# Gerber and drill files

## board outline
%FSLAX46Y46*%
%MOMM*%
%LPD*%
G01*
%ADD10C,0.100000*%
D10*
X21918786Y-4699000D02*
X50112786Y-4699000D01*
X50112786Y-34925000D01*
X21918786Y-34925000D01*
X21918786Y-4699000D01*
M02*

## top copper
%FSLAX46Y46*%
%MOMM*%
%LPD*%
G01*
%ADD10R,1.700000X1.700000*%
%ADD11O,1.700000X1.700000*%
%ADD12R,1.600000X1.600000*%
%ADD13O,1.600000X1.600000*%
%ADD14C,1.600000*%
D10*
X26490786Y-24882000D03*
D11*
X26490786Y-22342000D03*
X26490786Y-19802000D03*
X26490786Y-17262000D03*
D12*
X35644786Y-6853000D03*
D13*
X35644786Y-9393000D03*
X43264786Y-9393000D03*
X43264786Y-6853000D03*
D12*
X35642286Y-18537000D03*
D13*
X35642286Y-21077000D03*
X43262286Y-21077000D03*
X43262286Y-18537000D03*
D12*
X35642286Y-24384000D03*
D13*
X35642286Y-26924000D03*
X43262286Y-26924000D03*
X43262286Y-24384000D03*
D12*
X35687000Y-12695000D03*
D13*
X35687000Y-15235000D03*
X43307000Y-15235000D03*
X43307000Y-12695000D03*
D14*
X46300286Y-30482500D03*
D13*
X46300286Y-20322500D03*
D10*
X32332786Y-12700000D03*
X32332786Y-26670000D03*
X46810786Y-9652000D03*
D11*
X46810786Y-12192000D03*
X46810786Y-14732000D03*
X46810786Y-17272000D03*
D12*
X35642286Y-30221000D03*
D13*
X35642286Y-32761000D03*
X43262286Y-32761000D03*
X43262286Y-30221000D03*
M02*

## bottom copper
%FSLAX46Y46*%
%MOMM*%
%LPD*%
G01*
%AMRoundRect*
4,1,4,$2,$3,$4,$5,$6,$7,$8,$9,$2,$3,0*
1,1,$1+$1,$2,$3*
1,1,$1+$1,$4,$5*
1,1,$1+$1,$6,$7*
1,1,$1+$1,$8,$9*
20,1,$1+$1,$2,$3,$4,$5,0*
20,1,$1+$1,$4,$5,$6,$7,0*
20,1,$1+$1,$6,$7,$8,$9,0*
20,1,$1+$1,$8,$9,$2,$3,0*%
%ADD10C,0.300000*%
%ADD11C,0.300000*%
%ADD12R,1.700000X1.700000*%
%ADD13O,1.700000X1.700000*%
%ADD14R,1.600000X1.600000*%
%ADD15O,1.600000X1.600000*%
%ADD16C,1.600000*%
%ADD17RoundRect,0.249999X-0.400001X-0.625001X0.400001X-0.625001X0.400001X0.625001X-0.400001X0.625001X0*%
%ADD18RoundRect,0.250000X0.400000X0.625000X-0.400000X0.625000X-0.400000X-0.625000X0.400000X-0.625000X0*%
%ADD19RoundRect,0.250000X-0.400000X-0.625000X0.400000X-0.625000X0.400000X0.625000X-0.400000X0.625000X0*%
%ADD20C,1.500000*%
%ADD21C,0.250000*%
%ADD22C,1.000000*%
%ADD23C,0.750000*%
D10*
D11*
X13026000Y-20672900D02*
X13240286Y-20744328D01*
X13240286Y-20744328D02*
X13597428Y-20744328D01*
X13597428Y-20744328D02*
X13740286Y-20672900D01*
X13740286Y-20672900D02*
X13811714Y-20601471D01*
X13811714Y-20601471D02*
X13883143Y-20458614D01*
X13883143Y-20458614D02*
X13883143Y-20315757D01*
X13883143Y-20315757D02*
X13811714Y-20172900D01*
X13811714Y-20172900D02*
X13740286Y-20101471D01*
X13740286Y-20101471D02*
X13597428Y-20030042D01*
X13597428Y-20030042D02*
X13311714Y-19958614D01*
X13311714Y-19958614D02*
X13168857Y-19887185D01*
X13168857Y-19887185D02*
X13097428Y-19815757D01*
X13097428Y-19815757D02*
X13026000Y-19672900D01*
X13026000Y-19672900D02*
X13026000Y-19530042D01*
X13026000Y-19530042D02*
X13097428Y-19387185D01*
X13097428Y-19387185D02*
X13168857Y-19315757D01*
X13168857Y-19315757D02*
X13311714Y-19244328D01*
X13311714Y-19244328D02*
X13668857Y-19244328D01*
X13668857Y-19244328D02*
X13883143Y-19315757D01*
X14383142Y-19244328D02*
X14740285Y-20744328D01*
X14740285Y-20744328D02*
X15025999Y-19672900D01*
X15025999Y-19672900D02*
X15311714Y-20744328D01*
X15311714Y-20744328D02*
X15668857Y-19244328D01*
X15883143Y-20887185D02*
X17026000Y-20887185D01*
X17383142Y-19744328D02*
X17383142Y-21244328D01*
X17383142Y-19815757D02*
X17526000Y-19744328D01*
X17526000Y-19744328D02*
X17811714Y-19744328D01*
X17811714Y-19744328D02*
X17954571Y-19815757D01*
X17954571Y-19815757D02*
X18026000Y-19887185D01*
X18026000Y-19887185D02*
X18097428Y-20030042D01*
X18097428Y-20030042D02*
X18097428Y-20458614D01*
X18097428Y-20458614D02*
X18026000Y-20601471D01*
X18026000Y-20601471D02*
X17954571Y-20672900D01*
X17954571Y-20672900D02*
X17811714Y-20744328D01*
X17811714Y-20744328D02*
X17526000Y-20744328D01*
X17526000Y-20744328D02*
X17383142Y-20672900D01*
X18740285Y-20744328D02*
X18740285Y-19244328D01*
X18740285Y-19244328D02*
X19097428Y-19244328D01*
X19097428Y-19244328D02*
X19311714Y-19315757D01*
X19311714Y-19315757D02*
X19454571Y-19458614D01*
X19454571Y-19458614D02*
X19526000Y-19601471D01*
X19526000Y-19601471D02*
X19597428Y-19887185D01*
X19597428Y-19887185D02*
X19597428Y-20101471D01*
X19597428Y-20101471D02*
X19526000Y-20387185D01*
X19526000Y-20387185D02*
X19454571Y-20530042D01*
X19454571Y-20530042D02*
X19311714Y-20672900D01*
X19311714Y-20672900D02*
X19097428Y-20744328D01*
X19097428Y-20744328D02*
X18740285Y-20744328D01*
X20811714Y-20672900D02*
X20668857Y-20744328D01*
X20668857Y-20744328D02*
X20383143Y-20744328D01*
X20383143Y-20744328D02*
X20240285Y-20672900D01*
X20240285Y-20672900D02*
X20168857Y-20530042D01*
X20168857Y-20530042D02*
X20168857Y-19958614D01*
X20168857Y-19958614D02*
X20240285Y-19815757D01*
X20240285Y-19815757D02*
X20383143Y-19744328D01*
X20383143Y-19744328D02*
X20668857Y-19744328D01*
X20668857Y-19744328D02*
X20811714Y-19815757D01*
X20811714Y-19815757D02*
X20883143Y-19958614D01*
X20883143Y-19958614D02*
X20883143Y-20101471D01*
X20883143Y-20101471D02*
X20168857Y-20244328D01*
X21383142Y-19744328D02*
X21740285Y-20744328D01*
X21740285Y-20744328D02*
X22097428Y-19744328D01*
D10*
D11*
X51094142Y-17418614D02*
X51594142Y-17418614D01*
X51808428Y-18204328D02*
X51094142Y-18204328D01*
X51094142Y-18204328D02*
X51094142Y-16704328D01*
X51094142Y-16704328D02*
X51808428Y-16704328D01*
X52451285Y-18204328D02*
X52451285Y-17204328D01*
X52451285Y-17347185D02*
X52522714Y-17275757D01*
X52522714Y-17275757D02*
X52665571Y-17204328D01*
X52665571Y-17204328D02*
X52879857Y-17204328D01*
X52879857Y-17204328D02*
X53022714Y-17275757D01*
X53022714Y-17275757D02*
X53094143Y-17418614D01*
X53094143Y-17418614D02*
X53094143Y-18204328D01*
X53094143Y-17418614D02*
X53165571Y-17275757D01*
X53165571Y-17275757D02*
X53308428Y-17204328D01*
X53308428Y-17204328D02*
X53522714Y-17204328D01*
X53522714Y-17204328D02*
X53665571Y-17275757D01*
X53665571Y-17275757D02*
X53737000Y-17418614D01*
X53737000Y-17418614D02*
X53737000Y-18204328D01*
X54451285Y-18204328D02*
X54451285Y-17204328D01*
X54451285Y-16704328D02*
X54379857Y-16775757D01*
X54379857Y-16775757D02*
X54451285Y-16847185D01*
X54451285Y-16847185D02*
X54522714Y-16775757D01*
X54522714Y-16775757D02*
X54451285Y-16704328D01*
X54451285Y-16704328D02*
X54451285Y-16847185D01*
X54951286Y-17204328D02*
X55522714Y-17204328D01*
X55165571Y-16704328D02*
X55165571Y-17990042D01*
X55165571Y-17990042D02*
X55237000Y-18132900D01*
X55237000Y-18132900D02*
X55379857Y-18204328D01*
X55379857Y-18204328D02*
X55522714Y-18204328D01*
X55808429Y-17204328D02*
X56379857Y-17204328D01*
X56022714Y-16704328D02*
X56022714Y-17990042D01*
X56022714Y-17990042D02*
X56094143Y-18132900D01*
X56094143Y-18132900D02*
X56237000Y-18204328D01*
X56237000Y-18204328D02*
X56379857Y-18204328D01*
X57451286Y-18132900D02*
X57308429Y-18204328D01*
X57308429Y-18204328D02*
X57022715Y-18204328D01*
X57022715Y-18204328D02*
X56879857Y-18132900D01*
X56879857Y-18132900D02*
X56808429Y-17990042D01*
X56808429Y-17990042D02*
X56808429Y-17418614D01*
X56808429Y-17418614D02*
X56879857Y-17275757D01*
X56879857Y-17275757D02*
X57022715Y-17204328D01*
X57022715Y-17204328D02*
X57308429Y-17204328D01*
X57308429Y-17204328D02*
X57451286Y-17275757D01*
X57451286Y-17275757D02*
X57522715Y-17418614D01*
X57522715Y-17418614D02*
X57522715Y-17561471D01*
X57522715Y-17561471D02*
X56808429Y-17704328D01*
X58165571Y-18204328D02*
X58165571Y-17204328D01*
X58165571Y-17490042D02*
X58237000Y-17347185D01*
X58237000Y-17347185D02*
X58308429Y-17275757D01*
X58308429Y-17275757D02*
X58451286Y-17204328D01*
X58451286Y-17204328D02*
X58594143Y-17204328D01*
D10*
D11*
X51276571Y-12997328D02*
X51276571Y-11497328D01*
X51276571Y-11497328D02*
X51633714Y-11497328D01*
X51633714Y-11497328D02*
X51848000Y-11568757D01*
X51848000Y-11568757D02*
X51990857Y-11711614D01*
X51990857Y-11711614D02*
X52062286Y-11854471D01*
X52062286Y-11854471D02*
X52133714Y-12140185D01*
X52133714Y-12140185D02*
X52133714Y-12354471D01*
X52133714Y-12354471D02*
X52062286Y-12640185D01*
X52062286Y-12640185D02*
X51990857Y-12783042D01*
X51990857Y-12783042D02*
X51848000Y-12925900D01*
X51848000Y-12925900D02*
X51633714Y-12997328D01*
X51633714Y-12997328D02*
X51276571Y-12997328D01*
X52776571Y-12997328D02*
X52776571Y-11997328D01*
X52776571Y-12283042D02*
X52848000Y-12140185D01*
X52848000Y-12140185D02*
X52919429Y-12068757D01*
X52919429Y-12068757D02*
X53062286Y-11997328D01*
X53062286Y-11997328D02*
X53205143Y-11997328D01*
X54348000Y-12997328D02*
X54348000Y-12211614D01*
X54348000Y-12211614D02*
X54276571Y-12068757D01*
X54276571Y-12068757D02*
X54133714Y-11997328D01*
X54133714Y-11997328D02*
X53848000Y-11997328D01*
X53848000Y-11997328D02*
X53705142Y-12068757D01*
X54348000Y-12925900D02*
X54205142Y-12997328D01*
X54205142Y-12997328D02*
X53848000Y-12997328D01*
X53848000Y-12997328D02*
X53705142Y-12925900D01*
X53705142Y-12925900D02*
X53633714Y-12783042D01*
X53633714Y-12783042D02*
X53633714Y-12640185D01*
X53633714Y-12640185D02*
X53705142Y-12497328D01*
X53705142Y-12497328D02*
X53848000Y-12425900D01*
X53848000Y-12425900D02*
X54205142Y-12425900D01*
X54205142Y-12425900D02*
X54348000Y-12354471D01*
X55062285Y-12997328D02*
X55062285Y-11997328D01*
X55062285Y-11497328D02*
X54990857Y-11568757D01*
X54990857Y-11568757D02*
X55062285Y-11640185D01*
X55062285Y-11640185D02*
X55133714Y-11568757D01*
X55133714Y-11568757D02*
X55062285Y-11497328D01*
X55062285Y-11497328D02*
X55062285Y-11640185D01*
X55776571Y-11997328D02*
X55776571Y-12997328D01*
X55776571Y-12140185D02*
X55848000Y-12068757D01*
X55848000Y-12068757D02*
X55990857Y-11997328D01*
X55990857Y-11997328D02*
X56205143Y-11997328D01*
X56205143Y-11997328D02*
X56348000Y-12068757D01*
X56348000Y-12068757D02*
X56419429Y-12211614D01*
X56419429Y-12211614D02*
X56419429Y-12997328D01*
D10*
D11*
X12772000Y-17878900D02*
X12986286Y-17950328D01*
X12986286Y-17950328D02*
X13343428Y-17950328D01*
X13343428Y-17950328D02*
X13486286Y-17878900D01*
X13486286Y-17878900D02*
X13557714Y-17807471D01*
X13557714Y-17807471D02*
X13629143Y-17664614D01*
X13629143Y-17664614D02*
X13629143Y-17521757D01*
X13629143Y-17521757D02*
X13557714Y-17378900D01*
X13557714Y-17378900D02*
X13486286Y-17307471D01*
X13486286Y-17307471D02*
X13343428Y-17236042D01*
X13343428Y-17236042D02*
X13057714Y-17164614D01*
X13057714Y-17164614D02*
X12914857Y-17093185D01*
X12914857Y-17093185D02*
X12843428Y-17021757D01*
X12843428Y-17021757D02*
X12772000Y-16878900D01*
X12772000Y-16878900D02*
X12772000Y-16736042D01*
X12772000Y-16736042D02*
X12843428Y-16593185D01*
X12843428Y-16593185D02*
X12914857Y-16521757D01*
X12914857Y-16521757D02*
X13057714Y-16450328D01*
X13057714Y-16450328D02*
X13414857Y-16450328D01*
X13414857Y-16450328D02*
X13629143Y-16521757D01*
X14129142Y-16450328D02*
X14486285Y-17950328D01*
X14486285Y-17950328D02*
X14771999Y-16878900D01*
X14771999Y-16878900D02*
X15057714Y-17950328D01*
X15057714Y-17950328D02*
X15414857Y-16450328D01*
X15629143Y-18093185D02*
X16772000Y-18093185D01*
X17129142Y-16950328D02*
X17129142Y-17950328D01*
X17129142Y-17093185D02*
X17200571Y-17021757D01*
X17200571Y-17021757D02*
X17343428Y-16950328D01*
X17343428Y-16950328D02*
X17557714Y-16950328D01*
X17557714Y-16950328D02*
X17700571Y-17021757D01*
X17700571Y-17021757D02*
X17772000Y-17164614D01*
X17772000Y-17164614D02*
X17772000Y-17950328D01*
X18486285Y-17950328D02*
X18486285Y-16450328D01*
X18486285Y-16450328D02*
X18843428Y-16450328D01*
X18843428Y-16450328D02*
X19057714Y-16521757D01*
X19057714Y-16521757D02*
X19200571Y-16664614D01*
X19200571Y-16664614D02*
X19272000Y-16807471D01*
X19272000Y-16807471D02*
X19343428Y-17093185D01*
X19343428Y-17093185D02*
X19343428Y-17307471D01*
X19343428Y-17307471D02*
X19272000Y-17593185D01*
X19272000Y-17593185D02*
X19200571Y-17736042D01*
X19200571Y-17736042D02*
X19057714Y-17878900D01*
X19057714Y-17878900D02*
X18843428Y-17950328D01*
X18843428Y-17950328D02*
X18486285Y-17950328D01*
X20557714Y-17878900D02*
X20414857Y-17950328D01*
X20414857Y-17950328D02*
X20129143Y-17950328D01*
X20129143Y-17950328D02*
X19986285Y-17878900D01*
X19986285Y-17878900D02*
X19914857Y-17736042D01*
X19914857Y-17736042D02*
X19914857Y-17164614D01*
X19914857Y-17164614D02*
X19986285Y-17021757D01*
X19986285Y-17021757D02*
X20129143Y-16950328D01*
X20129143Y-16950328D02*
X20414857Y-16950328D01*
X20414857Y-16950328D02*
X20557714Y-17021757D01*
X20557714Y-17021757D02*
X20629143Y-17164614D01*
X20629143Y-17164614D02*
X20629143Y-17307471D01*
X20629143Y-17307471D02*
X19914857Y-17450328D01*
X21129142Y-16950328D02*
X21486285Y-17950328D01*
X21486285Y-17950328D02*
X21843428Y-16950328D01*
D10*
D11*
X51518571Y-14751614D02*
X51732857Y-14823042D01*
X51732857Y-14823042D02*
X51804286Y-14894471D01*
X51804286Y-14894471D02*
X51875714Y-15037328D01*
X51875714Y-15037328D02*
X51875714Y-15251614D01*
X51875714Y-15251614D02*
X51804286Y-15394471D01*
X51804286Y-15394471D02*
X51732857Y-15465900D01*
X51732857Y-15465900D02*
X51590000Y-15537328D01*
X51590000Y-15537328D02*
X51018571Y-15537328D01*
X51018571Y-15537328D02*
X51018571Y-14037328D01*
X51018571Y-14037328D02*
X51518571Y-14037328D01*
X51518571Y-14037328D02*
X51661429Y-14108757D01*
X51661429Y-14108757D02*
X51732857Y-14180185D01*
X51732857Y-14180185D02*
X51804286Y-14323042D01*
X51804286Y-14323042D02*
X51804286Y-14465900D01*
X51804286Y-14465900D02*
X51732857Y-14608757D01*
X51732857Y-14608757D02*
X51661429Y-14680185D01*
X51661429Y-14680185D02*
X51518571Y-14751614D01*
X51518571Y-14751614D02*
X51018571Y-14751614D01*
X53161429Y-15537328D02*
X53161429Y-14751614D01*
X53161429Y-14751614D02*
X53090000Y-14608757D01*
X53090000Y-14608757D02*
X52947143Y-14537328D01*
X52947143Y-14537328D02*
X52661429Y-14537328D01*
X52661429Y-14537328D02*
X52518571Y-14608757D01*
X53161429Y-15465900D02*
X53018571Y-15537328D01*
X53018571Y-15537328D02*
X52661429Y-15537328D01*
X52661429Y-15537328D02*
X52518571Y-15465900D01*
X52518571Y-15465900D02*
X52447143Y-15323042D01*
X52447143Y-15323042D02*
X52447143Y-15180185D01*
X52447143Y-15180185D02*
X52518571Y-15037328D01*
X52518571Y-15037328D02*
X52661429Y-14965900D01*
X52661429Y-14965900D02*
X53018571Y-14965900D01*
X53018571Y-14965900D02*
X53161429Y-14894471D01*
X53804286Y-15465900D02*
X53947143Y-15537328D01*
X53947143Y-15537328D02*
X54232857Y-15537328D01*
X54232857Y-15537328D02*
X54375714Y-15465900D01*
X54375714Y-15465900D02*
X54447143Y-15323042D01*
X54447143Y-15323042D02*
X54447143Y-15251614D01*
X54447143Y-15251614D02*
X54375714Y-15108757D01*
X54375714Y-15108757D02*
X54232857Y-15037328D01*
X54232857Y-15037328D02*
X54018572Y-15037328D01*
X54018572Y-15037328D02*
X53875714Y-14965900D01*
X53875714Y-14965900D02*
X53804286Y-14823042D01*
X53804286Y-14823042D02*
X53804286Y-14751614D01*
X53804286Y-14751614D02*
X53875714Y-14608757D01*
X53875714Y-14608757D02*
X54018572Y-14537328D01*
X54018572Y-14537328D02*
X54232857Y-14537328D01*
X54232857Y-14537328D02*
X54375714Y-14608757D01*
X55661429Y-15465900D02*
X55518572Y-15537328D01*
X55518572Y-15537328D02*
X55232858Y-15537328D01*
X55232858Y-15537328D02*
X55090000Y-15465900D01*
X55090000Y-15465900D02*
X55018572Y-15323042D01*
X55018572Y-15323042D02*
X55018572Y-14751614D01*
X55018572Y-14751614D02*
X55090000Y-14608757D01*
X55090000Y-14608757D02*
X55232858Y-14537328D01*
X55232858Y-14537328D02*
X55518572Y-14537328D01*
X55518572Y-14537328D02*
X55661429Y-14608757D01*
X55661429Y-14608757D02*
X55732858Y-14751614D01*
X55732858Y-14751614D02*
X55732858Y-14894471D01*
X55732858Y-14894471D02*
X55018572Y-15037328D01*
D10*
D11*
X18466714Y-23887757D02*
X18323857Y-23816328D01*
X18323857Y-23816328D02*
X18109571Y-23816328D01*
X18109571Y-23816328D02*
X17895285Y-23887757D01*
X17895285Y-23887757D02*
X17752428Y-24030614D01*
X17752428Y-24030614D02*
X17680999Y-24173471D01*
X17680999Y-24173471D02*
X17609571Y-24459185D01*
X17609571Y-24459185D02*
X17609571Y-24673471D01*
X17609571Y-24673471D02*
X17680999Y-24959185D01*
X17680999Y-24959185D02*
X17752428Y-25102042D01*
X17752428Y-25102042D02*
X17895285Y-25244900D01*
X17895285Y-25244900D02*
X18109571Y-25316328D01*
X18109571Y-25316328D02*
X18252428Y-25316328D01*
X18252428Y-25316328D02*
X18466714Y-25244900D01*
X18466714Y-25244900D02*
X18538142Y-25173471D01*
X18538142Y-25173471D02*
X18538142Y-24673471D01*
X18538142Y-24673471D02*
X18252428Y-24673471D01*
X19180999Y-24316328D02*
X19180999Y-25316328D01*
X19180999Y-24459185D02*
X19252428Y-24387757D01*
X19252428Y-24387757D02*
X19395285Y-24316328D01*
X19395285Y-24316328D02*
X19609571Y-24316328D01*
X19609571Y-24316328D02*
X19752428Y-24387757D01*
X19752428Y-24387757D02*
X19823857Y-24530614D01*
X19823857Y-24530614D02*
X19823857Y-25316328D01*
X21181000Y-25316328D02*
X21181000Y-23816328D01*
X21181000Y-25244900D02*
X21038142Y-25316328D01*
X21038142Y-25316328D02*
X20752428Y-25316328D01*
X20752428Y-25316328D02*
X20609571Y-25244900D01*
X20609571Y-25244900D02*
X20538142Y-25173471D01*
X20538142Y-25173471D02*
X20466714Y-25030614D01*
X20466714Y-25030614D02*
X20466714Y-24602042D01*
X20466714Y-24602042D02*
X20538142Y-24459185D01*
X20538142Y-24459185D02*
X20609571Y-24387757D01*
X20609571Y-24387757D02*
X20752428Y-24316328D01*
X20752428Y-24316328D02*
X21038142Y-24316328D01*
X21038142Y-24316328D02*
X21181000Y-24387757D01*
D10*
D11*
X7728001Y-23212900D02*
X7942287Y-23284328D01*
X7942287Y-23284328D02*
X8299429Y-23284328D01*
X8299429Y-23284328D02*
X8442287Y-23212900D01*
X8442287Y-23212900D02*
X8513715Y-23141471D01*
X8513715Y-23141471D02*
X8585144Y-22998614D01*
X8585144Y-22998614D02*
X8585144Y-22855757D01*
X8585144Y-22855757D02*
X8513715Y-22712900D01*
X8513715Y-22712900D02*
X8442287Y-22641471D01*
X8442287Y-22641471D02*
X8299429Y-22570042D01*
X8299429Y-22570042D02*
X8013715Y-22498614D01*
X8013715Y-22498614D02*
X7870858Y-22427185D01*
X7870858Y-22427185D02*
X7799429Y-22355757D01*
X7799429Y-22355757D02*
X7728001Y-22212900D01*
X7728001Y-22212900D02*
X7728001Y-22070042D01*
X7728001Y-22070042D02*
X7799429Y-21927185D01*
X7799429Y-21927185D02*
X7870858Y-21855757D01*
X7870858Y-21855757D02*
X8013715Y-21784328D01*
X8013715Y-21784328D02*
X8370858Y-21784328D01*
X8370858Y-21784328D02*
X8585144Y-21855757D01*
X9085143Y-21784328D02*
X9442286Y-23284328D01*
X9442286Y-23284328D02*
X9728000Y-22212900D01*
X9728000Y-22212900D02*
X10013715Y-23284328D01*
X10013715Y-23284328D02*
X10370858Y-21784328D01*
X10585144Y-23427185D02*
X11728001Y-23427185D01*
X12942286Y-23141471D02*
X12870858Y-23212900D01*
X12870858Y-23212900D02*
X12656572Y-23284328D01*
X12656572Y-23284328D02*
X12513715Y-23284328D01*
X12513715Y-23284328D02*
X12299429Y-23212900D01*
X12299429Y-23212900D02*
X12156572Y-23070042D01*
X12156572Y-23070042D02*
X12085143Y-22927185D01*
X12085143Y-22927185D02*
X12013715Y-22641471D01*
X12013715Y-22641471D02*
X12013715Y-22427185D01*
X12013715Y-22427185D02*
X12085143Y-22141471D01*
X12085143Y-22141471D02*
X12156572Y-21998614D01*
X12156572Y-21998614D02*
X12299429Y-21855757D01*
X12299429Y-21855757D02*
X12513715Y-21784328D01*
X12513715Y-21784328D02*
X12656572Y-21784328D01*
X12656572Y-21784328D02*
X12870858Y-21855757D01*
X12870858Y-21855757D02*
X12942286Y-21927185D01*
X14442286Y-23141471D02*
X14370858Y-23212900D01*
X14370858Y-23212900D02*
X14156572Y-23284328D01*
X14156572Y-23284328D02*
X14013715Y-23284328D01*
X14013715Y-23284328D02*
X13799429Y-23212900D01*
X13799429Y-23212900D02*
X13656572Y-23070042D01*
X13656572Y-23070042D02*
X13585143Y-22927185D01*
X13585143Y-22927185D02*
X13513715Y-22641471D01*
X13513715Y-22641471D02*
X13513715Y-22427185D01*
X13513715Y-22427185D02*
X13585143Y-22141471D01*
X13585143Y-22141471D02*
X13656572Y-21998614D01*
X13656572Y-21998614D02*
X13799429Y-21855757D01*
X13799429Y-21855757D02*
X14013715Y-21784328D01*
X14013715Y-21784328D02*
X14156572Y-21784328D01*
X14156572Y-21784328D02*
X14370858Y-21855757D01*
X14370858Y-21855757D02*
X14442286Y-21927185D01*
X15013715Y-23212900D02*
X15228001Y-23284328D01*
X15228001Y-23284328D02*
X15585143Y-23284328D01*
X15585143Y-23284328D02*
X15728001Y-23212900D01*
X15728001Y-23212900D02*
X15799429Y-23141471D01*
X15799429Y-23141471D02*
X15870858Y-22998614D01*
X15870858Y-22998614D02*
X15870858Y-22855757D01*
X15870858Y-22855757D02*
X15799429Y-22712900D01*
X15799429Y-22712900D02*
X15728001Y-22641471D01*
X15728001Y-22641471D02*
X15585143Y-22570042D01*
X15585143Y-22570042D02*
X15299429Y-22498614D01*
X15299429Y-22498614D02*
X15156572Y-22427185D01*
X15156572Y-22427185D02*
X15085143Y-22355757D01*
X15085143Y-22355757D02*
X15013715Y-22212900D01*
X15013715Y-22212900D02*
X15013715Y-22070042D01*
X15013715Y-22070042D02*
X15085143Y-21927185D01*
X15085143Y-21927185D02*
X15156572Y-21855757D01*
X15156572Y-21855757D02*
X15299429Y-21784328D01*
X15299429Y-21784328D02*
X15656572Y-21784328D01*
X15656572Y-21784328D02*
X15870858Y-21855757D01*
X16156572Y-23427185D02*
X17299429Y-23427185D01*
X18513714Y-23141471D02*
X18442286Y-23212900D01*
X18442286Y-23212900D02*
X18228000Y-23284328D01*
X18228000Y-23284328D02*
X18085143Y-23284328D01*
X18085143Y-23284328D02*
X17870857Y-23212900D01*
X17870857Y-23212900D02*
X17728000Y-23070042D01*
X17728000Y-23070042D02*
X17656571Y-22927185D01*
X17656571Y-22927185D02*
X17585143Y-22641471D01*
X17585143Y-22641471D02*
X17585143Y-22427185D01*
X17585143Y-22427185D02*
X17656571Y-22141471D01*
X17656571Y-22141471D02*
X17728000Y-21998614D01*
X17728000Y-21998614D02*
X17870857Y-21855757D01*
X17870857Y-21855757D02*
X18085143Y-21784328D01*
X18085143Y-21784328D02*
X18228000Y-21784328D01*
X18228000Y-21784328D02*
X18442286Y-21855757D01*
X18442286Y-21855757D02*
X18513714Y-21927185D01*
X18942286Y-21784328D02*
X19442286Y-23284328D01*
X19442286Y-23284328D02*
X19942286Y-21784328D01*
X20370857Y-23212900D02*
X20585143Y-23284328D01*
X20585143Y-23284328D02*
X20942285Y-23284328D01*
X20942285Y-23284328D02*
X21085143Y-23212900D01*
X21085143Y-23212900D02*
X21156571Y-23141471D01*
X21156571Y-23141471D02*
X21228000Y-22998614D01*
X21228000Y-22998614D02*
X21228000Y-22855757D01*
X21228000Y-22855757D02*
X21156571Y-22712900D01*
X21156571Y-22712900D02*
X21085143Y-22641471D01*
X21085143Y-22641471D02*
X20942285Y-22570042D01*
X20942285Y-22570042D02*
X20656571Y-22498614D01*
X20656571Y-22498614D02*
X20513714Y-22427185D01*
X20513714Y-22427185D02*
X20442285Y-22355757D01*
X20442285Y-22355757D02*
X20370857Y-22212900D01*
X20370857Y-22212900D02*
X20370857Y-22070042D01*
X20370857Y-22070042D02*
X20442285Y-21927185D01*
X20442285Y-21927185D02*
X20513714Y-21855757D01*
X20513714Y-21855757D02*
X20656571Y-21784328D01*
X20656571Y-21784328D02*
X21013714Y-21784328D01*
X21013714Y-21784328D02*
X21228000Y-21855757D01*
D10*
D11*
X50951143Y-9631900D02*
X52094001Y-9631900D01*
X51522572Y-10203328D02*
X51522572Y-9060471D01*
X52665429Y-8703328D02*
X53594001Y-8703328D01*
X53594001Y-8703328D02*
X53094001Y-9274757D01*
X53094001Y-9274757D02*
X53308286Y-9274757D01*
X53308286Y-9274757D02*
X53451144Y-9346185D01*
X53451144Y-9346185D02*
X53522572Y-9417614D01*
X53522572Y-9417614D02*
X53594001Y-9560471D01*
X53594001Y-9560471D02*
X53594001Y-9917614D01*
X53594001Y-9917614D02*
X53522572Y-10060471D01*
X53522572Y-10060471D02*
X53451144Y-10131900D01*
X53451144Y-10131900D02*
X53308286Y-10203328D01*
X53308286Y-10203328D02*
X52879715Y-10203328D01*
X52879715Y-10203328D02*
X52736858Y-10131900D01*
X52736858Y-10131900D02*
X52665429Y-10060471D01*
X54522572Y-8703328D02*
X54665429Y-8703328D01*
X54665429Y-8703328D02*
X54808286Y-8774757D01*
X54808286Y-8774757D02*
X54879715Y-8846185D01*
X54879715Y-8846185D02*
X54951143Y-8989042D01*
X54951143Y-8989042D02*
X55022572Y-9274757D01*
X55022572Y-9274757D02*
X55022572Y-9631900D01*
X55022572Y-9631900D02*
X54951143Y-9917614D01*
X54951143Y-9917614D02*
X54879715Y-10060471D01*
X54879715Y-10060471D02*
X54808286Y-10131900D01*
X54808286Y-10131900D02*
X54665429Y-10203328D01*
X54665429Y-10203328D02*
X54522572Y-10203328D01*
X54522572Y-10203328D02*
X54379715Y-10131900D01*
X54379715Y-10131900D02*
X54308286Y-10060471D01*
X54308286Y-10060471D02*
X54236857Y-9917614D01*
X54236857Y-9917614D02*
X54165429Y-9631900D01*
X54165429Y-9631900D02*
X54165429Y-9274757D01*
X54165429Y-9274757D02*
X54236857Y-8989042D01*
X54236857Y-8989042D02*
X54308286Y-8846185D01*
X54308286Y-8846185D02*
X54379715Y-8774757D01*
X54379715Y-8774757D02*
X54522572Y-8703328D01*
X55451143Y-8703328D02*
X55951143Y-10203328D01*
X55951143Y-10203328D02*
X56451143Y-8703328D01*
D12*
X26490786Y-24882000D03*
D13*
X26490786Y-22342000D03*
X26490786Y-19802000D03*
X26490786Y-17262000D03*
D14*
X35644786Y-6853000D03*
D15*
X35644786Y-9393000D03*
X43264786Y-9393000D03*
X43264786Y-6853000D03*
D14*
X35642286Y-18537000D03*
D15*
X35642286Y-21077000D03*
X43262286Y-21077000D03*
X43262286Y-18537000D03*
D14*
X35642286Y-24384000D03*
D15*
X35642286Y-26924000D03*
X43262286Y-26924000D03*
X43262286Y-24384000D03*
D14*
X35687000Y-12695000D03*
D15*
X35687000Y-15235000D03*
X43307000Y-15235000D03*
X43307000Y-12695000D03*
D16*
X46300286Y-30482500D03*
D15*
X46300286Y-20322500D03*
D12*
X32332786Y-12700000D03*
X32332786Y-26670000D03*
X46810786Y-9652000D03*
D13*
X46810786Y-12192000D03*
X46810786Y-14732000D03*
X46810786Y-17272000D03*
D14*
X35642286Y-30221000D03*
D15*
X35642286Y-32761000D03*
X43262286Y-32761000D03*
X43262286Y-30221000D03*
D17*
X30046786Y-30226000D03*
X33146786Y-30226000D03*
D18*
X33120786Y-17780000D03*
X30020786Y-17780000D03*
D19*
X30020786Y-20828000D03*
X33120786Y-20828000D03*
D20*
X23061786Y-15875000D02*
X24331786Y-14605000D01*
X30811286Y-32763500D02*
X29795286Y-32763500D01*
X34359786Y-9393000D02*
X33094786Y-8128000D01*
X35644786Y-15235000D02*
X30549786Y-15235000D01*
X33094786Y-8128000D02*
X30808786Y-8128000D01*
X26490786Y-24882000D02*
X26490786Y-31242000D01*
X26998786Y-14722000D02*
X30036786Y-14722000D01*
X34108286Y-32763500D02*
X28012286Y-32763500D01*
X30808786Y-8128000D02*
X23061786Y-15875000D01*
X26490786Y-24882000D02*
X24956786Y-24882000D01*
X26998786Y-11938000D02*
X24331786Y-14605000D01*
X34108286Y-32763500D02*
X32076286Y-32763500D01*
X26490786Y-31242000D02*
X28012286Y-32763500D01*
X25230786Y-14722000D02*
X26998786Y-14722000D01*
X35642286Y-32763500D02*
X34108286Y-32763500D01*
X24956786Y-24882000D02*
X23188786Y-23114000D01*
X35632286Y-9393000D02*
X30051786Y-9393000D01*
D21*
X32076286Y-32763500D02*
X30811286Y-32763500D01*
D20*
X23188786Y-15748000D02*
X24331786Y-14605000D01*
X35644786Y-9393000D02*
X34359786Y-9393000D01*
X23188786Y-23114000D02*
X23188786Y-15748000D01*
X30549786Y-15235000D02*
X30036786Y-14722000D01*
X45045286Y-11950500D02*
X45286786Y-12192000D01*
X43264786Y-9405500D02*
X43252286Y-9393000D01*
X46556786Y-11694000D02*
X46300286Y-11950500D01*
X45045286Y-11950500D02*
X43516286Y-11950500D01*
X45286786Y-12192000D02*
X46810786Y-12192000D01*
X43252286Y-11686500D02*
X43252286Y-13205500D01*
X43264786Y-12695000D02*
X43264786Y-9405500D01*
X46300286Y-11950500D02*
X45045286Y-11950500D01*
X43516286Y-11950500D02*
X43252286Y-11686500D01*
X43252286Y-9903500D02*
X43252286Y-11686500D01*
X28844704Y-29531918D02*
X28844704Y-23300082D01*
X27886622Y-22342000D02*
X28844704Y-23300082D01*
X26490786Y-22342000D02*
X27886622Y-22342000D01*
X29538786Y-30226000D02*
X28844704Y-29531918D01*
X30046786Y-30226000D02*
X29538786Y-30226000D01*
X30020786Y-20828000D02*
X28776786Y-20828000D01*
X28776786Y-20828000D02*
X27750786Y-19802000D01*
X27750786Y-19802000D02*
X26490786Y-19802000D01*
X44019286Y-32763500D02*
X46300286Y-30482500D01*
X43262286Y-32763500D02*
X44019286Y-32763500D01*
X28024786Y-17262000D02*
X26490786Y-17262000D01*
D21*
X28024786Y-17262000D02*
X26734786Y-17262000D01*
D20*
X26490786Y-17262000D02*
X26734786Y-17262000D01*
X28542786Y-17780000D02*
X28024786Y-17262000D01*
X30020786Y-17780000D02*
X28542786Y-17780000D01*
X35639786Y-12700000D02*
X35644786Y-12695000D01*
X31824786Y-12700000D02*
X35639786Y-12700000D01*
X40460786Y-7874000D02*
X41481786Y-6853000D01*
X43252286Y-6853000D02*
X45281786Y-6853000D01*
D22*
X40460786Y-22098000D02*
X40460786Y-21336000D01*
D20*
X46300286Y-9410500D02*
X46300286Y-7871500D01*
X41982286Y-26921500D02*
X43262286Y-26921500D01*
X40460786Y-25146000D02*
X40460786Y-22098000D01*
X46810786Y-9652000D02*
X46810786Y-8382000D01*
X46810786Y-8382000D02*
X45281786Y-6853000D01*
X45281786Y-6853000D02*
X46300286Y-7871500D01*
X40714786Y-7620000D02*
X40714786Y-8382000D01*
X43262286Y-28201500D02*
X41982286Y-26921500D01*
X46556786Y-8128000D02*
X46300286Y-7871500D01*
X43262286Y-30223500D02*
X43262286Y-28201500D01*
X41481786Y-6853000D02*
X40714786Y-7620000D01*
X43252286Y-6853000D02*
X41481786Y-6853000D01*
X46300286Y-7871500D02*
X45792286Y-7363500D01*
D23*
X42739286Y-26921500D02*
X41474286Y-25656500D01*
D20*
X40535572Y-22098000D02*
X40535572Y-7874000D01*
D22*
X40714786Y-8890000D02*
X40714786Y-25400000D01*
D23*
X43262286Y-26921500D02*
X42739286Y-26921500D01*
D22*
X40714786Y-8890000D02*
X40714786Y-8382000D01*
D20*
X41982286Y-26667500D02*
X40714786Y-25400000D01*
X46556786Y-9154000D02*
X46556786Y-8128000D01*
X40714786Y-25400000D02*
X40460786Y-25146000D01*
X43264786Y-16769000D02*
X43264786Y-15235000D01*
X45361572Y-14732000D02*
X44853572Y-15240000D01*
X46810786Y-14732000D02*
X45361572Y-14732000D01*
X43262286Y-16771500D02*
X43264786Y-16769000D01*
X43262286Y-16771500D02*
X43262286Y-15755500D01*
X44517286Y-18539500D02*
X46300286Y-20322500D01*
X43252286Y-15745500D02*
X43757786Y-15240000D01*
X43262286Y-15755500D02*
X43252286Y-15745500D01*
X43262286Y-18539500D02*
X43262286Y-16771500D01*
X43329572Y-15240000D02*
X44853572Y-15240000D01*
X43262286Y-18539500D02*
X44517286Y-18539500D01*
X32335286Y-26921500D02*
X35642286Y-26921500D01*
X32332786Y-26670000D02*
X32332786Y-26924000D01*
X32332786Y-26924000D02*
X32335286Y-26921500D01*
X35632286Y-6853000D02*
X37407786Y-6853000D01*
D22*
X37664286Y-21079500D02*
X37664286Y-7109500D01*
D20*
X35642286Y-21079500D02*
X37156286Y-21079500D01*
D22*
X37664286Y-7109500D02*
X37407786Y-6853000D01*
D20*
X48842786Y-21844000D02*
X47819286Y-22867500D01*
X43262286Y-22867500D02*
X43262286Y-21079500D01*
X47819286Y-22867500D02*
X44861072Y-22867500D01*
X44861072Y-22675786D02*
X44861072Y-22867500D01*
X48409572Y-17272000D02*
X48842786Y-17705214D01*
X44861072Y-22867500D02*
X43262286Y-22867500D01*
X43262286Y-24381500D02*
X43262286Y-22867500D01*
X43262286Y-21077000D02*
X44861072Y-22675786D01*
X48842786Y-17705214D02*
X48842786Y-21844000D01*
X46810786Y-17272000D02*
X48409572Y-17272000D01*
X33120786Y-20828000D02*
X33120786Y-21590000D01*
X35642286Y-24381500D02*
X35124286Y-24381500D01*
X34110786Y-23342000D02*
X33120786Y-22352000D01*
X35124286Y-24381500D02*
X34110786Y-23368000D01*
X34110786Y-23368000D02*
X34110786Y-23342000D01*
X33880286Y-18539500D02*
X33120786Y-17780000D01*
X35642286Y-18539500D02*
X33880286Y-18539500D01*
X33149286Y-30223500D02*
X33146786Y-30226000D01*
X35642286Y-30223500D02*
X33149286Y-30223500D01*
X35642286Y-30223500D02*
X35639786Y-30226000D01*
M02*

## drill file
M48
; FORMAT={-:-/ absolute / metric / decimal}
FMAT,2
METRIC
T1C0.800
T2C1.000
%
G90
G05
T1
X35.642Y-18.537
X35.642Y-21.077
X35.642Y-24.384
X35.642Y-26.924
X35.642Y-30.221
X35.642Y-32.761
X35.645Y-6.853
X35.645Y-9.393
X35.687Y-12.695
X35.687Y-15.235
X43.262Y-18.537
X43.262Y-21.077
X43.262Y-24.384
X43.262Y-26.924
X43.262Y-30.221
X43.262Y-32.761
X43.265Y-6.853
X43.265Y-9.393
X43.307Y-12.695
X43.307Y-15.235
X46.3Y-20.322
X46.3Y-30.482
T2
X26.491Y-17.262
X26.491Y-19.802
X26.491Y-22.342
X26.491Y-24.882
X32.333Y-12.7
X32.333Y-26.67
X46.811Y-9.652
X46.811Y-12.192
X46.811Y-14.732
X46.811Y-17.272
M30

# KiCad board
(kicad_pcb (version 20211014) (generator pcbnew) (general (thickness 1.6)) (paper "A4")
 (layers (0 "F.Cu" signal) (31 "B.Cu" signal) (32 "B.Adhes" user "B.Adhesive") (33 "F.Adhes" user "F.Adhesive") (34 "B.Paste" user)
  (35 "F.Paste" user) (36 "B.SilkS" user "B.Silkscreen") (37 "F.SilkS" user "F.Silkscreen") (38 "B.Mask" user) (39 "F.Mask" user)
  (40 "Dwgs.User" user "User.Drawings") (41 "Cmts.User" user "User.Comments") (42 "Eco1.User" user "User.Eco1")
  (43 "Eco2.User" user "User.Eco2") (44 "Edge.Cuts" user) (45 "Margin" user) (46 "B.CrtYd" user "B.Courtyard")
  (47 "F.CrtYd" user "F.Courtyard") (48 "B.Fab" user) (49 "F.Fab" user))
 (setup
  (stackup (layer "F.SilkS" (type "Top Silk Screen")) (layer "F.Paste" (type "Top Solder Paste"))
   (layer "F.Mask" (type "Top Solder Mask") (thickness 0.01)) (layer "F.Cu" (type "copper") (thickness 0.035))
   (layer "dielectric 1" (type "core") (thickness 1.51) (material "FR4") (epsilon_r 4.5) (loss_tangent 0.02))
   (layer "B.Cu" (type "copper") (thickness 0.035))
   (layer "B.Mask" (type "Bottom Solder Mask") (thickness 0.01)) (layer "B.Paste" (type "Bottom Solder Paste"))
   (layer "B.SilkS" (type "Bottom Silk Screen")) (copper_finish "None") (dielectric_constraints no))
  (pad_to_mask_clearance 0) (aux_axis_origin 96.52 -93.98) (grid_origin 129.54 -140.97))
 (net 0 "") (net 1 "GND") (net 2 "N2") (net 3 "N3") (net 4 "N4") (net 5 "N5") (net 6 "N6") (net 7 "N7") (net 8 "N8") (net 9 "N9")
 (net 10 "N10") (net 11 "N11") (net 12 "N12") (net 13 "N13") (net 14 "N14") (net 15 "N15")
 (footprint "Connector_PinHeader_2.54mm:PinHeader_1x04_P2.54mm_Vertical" (layer "F.Cu") (at 26.490786 24.882 180)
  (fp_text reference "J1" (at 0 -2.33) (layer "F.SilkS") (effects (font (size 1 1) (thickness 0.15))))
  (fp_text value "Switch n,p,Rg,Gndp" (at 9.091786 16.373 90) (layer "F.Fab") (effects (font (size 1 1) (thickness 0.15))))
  (pad "1" thru_hole rect (at 0 0 180) (size 1.7 1.7) (drill 1) (layers *.Cu *.Mask) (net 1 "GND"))
  (pad "2" thru_hole oval (at 0 2.54 180) (size 1.7 1.7) (drill 1) (layers *.Cu *.Mask) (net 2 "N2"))
  (pad "3" thru_hole oval (at 0 5.08 180) (size 1.7 1.7) (drill 1) (layers *.Cu *.Mask) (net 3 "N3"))
  (pad "4" thru_hole oval (at 0 7.62 180) (size 1.7 1.7) (drill 1) (layers *.Cu *.Mask) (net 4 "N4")))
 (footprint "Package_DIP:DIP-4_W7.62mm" (layer "F.Cu") (at 35.644786 6.853)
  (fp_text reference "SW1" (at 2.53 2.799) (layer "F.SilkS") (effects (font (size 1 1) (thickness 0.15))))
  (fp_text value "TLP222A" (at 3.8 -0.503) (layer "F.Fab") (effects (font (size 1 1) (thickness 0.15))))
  (pad "1" thru_hole rect locked (at 0 0) (size 1.6 1.6) (drill 0.8) (layers *.Cu *.Mask) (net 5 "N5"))
  (pad "2" thru_hole oval locked (at 0 2.54) (size 1.6 1.6) (drill 0.8) (layers *.Cu *.Mask) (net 1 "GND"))
  (pad "3" thru_hole oval locked (at 7.62 2.54) (size 1.6 1.6) (drill 0.8) (layers *.Cu *.Mask) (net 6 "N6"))
  (pad "4" thru_hole oval locked (at 7.62 0) (size 1.6 1.6) (drill 0.8) (layers *.Cu *.Mask) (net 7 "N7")))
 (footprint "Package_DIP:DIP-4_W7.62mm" (layer "F.Cu") (at 35.642286 18.537)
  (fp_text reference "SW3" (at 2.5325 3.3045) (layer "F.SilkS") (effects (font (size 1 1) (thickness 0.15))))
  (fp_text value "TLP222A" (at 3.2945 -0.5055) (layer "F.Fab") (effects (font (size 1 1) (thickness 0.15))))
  (pad "1" thru_hole rect locked (at 0 0) (size 1.6 1.6) (drill 0.8) (layers *.Cu *.Mask) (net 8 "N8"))
  (pad "2" thru_hole oval locked (at 0 2.54) (size 1.6 1.6) (drill 0.8) (layers *.Cu *.Mask) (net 5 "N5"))
  (pad "3" thru_hole oval locked (at 7.62 2.54) (size 1.6 1.6) (drill 0.8) (layers *.Cu *.Mask) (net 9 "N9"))
  (pad "4" thru_hole oval locked (at 7.62 0) (size 1.6 1.6) (drill 0.8) (layers *.Cu *.Mask) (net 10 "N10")))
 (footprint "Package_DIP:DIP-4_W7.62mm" (layer "F.Cu") (at 35.642286 24.384)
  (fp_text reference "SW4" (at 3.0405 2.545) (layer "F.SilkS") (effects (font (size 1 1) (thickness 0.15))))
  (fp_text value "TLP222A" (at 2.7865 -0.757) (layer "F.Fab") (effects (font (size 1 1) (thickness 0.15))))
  (pad "1" thru_hole rect locked (at 0 0) (size 1.6 1.6) (drill 0.8) (layers *.Cu *.Mask) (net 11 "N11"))
  (pad "2" thru_hole oval locked (at 0 2.54) (size 1.6 1.6) (drill 0.8) (layers *.Cu *.Mask) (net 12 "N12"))
  (pad "3" thru_hole oval locked (at 7.62 2.54) (size 1.6 1.6) (drill 0.8) (layers *.Cu *.Mask) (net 7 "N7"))
  (pad "4" thru_hole oval locked (at 7.62 0) (size 1.6 1.6) (drill 0.8) (layers *.Cu *.Mask) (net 9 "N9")))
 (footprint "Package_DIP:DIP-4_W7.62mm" (layer "F.Cu") (at 35.687 12.695)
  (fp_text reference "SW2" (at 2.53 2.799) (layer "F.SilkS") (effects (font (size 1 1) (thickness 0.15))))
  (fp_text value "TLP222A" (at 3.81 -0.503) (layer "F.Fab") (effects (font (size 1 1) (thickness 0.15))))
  (pad "1" thru_hole rect locked (at 0 0) (size 1.6 1.6) (drill 0.8) (layers *.Cu *.Mask) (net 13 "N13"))
  (pad "2" thru_hole oval locked (at 0 2.54) (size 1.6 1.6) (drill 0.8) (layers *.Cu *.Mask) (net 1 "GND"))
  (pad "3" thru_hole oval locked (at 7.62 2.54) (size 1.6 1.6) (drill 0.8) (layers *.Cu *.Mask) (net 10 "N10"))
  (pad "4" thru_hole oval locked (at 7.62 0) (size 1.6 1.6) (drill 0.8) (layers *.Cu *.Mask) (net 6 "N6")))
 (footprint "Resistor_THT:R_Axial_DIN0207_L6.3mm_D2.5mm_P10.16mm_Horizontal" (layer "F.Cu") (at 46.300286 30.4825 90)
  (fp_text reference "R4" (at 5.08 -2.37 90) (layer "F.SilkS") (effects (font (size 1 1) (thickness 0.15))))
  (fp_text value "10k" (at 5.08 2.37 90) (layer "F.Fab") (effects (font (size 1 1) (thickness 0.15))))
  (pad "1" thru_hole circle locked (at 0 0 90) (size 1.6 1.6) (drill 0.8) (layers *.Cu *.Mask) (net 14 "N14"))
  (pad "2" thru_hole oval locked (at 10.16 0 90) (size 1.6 1.6) (drill 0.8) (layers *.Cu *.Mask) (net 10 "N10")))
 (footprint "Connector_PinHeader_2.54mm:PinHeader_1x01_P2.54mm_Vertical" (layer "F.Cu") (at 32.332786 12.7)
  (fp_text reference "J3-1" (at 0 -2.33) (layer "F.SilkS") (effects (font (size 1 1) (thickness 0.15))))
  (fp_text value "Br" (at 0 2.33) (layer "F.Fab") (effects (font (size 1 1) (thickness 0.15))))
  (pad "1" thru_hole rect (at 0 0) (size 1.7 1.7) (drill 1) (layers *.Cu *.Mask) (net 13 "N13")))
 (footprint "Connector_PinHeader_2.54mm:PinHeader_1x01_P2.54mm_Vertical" (layer "F.Cu") (at 32.332786 26.67)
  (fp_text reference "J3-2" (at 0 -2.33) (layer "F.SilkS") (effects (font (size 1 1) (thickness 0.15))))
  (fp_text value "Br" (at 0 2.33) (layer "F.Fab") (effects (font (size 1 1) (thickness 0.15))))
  (pad "1" thru_hole rect (at 0 0) (size 1.7 1.7) (drill 1) (layers *.Cu *.Mask) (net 12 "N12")))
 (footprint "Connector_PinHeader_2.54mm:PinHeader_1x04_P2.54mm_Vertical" (layer "F.Cu") (at 46.810786 9.652)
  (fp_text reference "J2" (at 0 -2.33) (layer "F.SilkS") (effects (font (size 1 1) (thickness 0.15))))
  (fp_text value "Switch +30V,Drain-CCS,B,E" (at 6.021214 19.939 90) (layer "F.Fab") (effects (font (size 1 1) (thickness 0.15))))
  (pad "1" thru_hole rect (at 0 0) (size 1.7 1.7) (drill 1) (layers *.Cu *.Mask) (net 7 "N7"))
  (pad "2" thru_hole oval (at 0 2.54) (size 1.7 1.7) (drill 1) (layers *.Cu *.Mask) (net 6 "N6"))
  (pad "3" thru_hole oval (at 0 5.08) (size 1.7 1.7) (drill 1) (layers *.Cu *.Mask) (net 10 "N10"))
  (pad "4" thru_hole oval (at 0 7.62) (size 1.7 1.7) (drill 1) (layers *.Cu *.Mask) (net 9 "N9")))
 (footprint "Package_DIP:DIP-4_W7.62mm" (layer "F.Cu") (at 35.642286 30.221)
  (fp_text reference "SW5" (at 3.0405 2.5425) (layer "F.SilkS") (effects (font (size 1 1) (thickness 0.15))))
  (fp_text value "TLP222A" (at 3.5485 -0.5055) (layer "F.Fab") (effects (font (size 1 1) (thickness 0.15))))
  (pad "1" thru_hole rect (at 0 0) (size 1.6 1.6) (drill 0.8) (layers *.Cu *.Mask) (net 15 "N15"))
  (pad "2" thru_hole oval (at 0 2.54) (size 1.6 1.6) (drill 0.8) (layers *.Cu *.Mask) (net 1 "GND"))
  (pad "3" thru_hole oval (at 7.62 2.54) (size 1.6 1.6) (drill 0.8) (layers *.Cu *.Mask) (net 14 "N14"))
  (pad "4" thru_hole oval (at 7.62 0) (size 1.6 1.6) (drill 0.8) (layers *.Cu *.Mask) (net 7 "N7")))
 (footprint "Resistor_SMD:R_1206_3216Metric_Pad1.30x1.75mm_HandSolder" (layer "B.Cu") (at 31.596786 30.226)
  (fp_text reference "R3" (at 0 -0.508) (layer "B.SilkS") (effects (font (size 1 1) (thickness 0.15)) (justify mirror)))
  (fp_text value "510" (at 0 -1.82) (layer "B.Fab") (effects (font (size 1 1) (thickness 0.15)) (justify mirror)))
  (pad "1" smd roundrect locked (at -1.55 0) (size 1.3 1.75) (layers "B.Cu" "B.Paste" "B.Mask") (roundrect_rratio 0.1923069231) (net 2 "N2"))
  (pad "2" smd roundrect locked (at 1.55 0) (size 1.3 1.75) (layers "B.Cu" "B.Paste" "B.Mask") (roundrect_rratio 0.1923069231)
   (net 15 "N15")))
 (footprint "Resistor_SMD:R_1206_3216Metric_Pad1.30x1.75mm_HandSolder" (layer "B.Cu") (at 31.570786 17.78 180)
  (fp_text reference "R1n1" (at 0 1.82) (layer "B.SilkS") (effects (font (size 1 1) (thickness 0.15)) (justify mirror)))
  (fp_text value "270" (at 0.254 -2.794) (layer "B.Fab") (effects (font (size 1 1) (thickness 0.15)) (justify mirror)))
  (pad "1" smd roundrect (at -1.55 0 180) (size 1.3 1.75) (layers "B.Cu" "B.Paste" "B.Mask") (roundrect_rratio 0.192308) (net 8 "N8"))
  (pad "2" smd roundrect (at 1.55 0 180) (size 1.3 1.75) (layers "B.Cu" "B.Paste" "B.Mask") (roundrect_rratio 0.192308) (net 4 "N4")))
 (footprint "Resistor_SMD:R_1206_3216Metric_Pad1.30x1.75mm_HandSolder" (layer "B.Cu") (at 31.570786 20.828)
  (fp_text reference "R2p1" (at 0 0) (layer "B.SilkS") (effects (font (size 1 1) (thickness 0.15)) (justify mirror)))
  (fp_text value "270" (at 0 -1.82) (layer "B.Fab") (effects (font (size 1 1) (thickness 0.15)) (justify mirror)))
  (pad "1" smd roundrect (at -1.55 0) (size 1.3 1.75) (layers "B.Cu" "B.Paste" "B.Mask") (roundrect_rratio 0.192308) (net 3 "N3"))
  (pad "2" smd roundrect (at 1.55 0) (size 1.3 1.75) (layers "B.Cu" "B.Paste" "B.Mask") (roundrect_rratio 0.192308) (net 11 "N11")))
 (gr_rect (start 21.918786 4.699) (end 50.112786 34.925) (layer "Edge.Cuts") (width 0.1) (fill none))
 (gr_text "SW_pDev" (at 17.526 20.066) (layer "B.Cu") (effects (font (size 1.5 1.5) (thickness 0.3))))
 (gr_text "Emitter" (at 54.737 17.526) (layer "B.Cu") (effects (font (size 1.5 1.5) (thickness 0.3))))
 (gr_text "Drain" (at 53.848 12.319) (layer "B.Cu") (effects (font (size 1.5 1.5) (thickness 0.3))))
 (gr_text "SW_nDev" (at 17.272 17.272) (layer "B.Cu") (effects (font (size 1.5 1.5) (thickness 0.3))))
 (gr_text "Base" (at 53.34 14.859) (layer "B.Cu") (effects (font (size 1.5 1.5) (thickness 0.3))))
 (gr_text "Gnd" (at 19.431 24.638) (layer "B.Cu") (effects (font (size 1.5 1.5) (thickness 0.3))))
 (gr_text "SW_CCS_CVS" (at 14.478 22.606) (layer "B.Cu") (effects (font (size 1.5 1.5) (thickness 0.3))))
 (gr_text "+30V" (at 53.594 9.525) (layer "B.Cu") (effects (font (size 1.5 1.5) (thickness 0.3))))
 (segment (start 23.061786 15.875) (end 24.331786 14.605) (width 1.5) (layer "B.Cu") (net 1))
 (segment (start 30.811286 32.7635) (end 29.795286 32.7635) (width 1.5) (layer "B.Cu") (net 1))
 (segment (start 34.359786 9.393) (end 33.094786 8.128) (width 1.5) (layer "B.Cu") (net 1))
 (segment (start 35.644786 15.235) (end 30.549786 15.235) (width 1.5) (layer "B.Cu") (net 1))
 (segment (start 33.094786 8.128) (end 30.808786 8.128) (width 1.5) (layer "B.Cu") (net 1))
 (segment (start 26.490786 24.882) (end 26.490786 31.242) (width 1.5) (layer "B.Cu") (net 1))
 (segment (start 26.998786 14.722) (end 30.036786 14.722) (width 1.5) (layer "B.Cu") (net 1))
 (segment (start 34.108286 32.7635) (end 28.012286 32.7635) (width 1.5) (layer "B.Cu") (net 1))
 (segment (start 30.808786 8.128) (end 23.061786 15.875) (width 1.5) (layer "B.Cu") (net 1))
 (segment (start 26.490786 24.882) (end 24.956786 24.882) (width 1.5) (layer "B.Cu") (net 1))
 (segment (start 26.998786 11.938) (end 24.331786 14.605) (width 1.5) (layer "B.Cu") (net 1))
 (segment (start 34.108286 32.7635) (end 32.076286 32.7635) (width 1.5) (layer "B.Cu") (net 1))
 (segment (start 26.490786 31.242) (end 28.012286 32.7635) (width 1.5) (layer "B.Cu") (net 1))
 (segment (start 25.230786 14.722) (end 26.998786 14.722) (width 1.5) (layer "B.Cu") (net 1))
 (segment (start 35.642286 32.7635) (end 34.108286 32.7635) (width 1.5) (layer "B.Cu") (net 1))
 (segment (start 24.956786 24.882) (end 23.188786 23.114) (width 1.5) (layer "B.Cu") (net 1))
 (segment (start 35.632286 9.393) (end 30.051786 9.393) (width 1.5) (layer "B.Cu") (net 1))
 (segment (start 32.076286 32.7635) (end 30.811286 32.7635) (width 0.25) (layer "B.Cu") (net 1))
 (segment (start 23.188786 15.748) (end 24.331786 14.605) (width 1.5) (layer "B.Cu") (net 1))
 (segment (start 35.644786 9.393) (end 34.359786 9.393) (width 1.5) (layer "B.Cu") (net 1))
 (segment (start 23.188786 23.114) (end 23.188786 15.748) (width 1.5) (layer "B.Cu") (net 1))
 (segment (start 30.549786 15.235) (end 30.036786 14.722) (width 1.5) (layer "B.Cu") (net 1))
 (segment (start 45.045286 11.9505) (end 45.286786 12.192) (width 1.5) (layer "B.Cu") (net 6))
 (segment (start 43.264786 9.4055) (end 43.252286 9.393) (width 1.5) (layer "B.Cu") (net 6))
 (segment (start 46.556786 11.694) (end 46.300286 11.9505) (width 1.5) (layer "B.Cu") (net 6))
 (segment (start 45.045286 11.9505) (end 43.516286 11.9505) (width 1.5) (layer "B.Cu") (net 6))
 (segment (start 45.286786 12.192) (end 46.810786 12.192) (width 1.5) (layer "B.Cu") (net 6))
 (segment (start 43.252286 11.6865) (end 43.252286 13.2055) (width 1.5) (layer "B.Cu") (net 6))
 (segment (start 43.264786 12.695) (end 43.264786 9.4055) (width 1.5) (layer "B.Cu") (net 6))
 (segment (start 46.300286 11.9505) (end 45.045286 11.9505) (width 1.5) (layer "B.Cu") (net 6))
 (segment (start 43.516286 11.9505) (end 43.252286 11.6865) (width 1.5) (layer "B.Cu") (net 6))
 (segment (start 43.252286 9.9035) (end 43.252286 11.6865) (width 1.5) (layer "B.Cu") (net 6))
 (segment (start 28.844704 29.531918) (end 28.844704 23.300082) (width 1.5) (layer "B.Cu") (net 2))
 (segment (start 27.886622 22.342) (end 28.844704 23.300082) (width 1.5) (layer "B.Cu") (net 2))
 (segment (start 26.490786 22.342) (end 27.886622 22.342) (width 1.5) (layer "B.Cu") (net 2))
 (segment (start 29.538786 30.226) (end 28.844704 29.531918) (width 1.5) (layer "B.Cu") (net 2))
 (segment (start 30.046786 30.226) (end 29.538786 30.226) (width 1.5) (layer "B.Cu") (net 2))
 (segment (start 30.020786 20.828) (end 28.776786 20.828) (width 1.5) (layer "B.Cu") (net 3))
 (segment (start 28.776786 20.828) (end 27.750786 19.802) (width 1.5) (layer "B.Cu") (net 3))
 (segment (start 27.750786 19.802) (end 26.490786 19.802) (width 1.5) (layer "B.Cu") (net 3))
 (segment (start 44.019286 32.7635) (end 46.300286 30.4825) (width 1.5) (layer "B.Cu") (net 14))
 (segment (start 43.262286 32.7635) (end 44.019286 32.7635) (width 1.5) (layer "B.Cu") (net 14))
 (segment (start 28.024786 17.262) (end 26.490786 17.262) (width 1.5) (layer "B.Cu") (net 4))
 (segment (start 28.024786 17.262) (end 26.734786 17.262) (width 0.25) (layer "B.Cu") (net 4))
 (segment (start 26.490786 17.262) (end 26.734786 17.262) (width 1.5) (layer "B.Cu") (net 4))
 (segment (start 28.542786 17.78) (end 28.024786 17.262) (width 1.5) (layer "B.Cu") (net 4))
 (segment (start 30.020786 17.78) (end 28.542786 17.78) (width 1.5) (layer "B.Cu") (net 4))
 (segment (start 35.639786 12.7) (end 35.644786 12.695) (width 1.5) (layer "B.Cu") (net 13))
 (segment (start 31.824786 12.7) (end 35.639786 12.7) (width 1.5) (layer "B.Cu") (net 13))
 (segment (start 40.460786 7.874) (end 41.481786 6.853) (width 1.5) (layer "B.Cu") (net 7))
 (segment (start 43.252286 6.853) (end 45.281786 6.853) (width 1.5) (layer "B.Cu") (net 7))
 (segment (start 40.460786 22.098) (end 40.460786 21.336) (width 1) (layer "B.Cu") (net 7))
 (segment (start 46.300286 9.4105) (end 46.300286 7.8715) (width 1.5) (layer "B.Cu") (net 7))
 (segment (start 41.982286 26.9215) (end 43.262286 26.9215) (width 1.5) (layer "B.Cu") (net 7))
 (segment (start 40.460786 25.146) (end 40.460786 22.098) (width 1.5) (layer "B.Cu") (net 7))
 (segment (start 46.810786 9.652) (end 46.810786 8.382) (width 1.5) (layer "B.Cu") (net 7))
 (segment (start 46.810786 8.382) (end 45.281786 6.853) (width 1.5) (layer "B.Cu") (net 7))
 (segment (start 45.281786 6.853) (end 46.300286 7.8715) (width 1.5) (layer "B.Cu") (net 7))
 (segment (start 40.714786 7.62) (end 40.714786 8.382) (width 1.5) (layer "B.Cu") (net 7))
 (segment (start 43.262286 28.2015) (end 41.982286 26.9215) (width 1.5) (layer "B.Cu") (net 7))
 (segment (start 46.556786 8.128) (end 46.300286 7.8715) (width 1.5) (layer "B.Cu") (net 7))
 (segment (start 43.262286 30.2235) (end 43.262286 28.2015) (width 1.5) (layer "B.Cu") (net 7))
 (segment (start 41.481786 6.853) (end 40.714786 7.62) (width 1.5) (layer "B.Cu") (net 7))
 (segment (start 43.252286 6.853) (end 41.481786 6.853) (width 1.5) (layer "B.Cu") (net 7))
 (segment (start 46.300286 7.8715) (end 45.792286 7.3635) (width 1.5) (layer "B.Cu") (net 7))
 (segment (start 42.739286 26.9215) (end 41.474286 25.6565) (width 0.75) (layer "B.Cu") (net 7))
 (segment (start 40.535572 22.098) (end 40.535572 7.874) (width 1.5) (layer "B.Cu") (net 7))
 (segment (start 40.714786 8.89) (end 40.714786 25.4) (width 1) (layer "B.Cu") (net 7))
 (segment (start 43.262286 26.9215) (end 42.739286 26.9215) (width 0.75) (layer "B.Cu") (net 7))
 (segment (start 40.714786 8.89) (end 40.714786 8.382) (width 1) (layer "B.Cu") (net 7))
 (segment (start 41.982286 26.6675) (end 40.714786 25.4) (width 1.5) (layer "B.Cu") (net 7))
 (segment (start 46.556786 9.154) (end 46.556786 8.128) (width 1.5) (layer "B.Cu") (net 7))
 (segment (start 40.714786 25.4) (end 40.460786 25.146) (width 1.5) (layer "B.Cu") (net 7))
 (segment (start 43.264786 16.769) (end 43.264786 15.235) (width 1.5) (layer "B.Cu") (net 10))
 (segment (start 45.361572 14.732) (end 44.853572 15.24) (width 1.5) (layer "B.Cu") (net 10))
 (segment (start 46.810786 14.732) (end 45.361572 14.732) (width 1.5) (layer "B.Cu") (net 10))
 (segment (start 43.262286 16.7715) (end 43.264786 16.769) (width 1.5) (layer "B.Cu") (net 10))
 (segment (start 43.262286 16.7715) (end 43.262286 15.7555) (width 1.5) (layer "B.Cu") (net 10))
 (segment (start 44.517286 18.5395) (end 46.300286 20.3225) (width 1.5) (layer "B.Cu") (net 10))
 (segment (start 43.252286 15.7455) (end 43.757786 15.24) (width 1.5) (layer "B.Cu") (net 10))
 (segment (start 43.262286 15.7555) (end 43.252286 15.7455) (width 1.5) (layer "B.Cu") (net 10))
 (segment (start 43.262286 18.5395) (end 43.262286 16.7715) (width 1.5) (layer "B.Cu") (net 10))
 (segment (start 43.329572 15.24) (end 44.853572 15.24) (width 1.5) (layer "B.Cu") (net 10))
 (segment (start 43.262286 18.5395) (end 44.517286 18.5395) (width 1.5) (layer "B.Cu") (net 10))
 (segment (start 32.335286 26.9215) (end 35.642286 26.9215) (width 1.5) (layer "B.Cu") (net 12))
 (segment (start 32.332786 26.67) (end 32.332786 26.924) (width 1.5) (layer "B.Cu") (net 12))
 (segment (start 32.332786 26.924) (end 32.335286 26.9215) (width 1.5) (layer "B.Cu") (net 12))
 (segment (start 35.632286 6.853) (end 37.407786 6.853) (width 1.5) (layer "B.Cu") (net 5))
 (segment (start 37.664286 21.0795) (end 37.664286 7.1095) (width 1) (layer "B.Cu") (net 5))
 (segment (start 35.642286 21.0795) (end 37.156286 21.0795) (width 1.5) (layer "B.Cu") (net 5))
 (segment (start 37.664286 7.1095) (end 37.407786 6.853) (width 1) (layer "B.Cu") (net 5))
 (segment (start 48.842786 21.844) (end 47.819286 22.8675) (width 1.5) (layer "B.Cu") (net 9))
 (segment (start 43.262286 22.8675) (end 43.262286 21.0795) (width 1.5) (layer "B.Cu") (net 9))
 (segment (start 47.819286 22.8675) (end 44.861072 22.8675) (width 1.5) (layer "B.Cu") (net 9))
 (segment (start 44.861072 22.675786) (end 44.861072 22.8675) (width 1.5) (layer "B.Cu") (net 9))
 (segment (start 48.409572 17.272) (end 48.842786 17.705214) (width 1.5) (layer "B.Cu") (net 9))
 (segment (start 44.861072 22.8675) (end 43.262286 22.8675) (width 1.5) (layer "B.Cu") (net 9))
 (segment (start 43.262286 24.3815) (end 43.262286 22.8675) (width 1.5) (layer "B.Cu") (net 9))
 (segment (start 43.262286 21.077) (end 44.861072 22.675786) (width 1.5) (layer "B.Cu") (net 9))
 (segment (start 48.842786 17.705214) (end 48.842786 21.844) (width 1.5) (layer "B.Cu") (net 9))
 (segment (start 46.810786 17.272) (end 48.409572 17.272) (width 1.5) (layer "B.Cu") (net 9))
 (segment (start 33.120786 20.828) (end 33.120786 21.59) (width 1.5) (layer "B.Cu") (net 11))
 (segment (start 35.642286 24.3815) (end 35.124286 24.3815) (width 1.5) (layer "B.Cu") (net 11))
 (segment (start 34.110786 23.342) (end 33.120786 22.352) (width 1.5) (layer "B.Cu") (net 11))
 (segment (start 35.124286 24.3815) (end 34.110786 23.368) (width 1.5) (layer "B.Cu") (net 11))
 (segment (start 34.110786 23.368) (end 34.110786 23.342) (width 1.5) (layer "B.Cu") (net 11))
 (segment (start 33.880286 18.5395) (end 33.120786 17.78) (width 1.5) (layer "B.Cu") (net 8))
 (segment (start 35.642286 18.5395) (end 33.880286 18.5395) (width 1.5) (layer "B.Cu") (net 8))
 (segment (start 33.149286 30.2235) (end 33.146786 30.226) (width 1.5) (layer "B.Cu") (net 15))
 (segment (start 35.642286 30.2235) (end 33.149286 30.2235) (width 1.5) (layer "B.Cu") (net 15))
 (segment (start 35.642286 30.2235) (end 35.639786 30.226) (width 1.5) (layer "B.Cu") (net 15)))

